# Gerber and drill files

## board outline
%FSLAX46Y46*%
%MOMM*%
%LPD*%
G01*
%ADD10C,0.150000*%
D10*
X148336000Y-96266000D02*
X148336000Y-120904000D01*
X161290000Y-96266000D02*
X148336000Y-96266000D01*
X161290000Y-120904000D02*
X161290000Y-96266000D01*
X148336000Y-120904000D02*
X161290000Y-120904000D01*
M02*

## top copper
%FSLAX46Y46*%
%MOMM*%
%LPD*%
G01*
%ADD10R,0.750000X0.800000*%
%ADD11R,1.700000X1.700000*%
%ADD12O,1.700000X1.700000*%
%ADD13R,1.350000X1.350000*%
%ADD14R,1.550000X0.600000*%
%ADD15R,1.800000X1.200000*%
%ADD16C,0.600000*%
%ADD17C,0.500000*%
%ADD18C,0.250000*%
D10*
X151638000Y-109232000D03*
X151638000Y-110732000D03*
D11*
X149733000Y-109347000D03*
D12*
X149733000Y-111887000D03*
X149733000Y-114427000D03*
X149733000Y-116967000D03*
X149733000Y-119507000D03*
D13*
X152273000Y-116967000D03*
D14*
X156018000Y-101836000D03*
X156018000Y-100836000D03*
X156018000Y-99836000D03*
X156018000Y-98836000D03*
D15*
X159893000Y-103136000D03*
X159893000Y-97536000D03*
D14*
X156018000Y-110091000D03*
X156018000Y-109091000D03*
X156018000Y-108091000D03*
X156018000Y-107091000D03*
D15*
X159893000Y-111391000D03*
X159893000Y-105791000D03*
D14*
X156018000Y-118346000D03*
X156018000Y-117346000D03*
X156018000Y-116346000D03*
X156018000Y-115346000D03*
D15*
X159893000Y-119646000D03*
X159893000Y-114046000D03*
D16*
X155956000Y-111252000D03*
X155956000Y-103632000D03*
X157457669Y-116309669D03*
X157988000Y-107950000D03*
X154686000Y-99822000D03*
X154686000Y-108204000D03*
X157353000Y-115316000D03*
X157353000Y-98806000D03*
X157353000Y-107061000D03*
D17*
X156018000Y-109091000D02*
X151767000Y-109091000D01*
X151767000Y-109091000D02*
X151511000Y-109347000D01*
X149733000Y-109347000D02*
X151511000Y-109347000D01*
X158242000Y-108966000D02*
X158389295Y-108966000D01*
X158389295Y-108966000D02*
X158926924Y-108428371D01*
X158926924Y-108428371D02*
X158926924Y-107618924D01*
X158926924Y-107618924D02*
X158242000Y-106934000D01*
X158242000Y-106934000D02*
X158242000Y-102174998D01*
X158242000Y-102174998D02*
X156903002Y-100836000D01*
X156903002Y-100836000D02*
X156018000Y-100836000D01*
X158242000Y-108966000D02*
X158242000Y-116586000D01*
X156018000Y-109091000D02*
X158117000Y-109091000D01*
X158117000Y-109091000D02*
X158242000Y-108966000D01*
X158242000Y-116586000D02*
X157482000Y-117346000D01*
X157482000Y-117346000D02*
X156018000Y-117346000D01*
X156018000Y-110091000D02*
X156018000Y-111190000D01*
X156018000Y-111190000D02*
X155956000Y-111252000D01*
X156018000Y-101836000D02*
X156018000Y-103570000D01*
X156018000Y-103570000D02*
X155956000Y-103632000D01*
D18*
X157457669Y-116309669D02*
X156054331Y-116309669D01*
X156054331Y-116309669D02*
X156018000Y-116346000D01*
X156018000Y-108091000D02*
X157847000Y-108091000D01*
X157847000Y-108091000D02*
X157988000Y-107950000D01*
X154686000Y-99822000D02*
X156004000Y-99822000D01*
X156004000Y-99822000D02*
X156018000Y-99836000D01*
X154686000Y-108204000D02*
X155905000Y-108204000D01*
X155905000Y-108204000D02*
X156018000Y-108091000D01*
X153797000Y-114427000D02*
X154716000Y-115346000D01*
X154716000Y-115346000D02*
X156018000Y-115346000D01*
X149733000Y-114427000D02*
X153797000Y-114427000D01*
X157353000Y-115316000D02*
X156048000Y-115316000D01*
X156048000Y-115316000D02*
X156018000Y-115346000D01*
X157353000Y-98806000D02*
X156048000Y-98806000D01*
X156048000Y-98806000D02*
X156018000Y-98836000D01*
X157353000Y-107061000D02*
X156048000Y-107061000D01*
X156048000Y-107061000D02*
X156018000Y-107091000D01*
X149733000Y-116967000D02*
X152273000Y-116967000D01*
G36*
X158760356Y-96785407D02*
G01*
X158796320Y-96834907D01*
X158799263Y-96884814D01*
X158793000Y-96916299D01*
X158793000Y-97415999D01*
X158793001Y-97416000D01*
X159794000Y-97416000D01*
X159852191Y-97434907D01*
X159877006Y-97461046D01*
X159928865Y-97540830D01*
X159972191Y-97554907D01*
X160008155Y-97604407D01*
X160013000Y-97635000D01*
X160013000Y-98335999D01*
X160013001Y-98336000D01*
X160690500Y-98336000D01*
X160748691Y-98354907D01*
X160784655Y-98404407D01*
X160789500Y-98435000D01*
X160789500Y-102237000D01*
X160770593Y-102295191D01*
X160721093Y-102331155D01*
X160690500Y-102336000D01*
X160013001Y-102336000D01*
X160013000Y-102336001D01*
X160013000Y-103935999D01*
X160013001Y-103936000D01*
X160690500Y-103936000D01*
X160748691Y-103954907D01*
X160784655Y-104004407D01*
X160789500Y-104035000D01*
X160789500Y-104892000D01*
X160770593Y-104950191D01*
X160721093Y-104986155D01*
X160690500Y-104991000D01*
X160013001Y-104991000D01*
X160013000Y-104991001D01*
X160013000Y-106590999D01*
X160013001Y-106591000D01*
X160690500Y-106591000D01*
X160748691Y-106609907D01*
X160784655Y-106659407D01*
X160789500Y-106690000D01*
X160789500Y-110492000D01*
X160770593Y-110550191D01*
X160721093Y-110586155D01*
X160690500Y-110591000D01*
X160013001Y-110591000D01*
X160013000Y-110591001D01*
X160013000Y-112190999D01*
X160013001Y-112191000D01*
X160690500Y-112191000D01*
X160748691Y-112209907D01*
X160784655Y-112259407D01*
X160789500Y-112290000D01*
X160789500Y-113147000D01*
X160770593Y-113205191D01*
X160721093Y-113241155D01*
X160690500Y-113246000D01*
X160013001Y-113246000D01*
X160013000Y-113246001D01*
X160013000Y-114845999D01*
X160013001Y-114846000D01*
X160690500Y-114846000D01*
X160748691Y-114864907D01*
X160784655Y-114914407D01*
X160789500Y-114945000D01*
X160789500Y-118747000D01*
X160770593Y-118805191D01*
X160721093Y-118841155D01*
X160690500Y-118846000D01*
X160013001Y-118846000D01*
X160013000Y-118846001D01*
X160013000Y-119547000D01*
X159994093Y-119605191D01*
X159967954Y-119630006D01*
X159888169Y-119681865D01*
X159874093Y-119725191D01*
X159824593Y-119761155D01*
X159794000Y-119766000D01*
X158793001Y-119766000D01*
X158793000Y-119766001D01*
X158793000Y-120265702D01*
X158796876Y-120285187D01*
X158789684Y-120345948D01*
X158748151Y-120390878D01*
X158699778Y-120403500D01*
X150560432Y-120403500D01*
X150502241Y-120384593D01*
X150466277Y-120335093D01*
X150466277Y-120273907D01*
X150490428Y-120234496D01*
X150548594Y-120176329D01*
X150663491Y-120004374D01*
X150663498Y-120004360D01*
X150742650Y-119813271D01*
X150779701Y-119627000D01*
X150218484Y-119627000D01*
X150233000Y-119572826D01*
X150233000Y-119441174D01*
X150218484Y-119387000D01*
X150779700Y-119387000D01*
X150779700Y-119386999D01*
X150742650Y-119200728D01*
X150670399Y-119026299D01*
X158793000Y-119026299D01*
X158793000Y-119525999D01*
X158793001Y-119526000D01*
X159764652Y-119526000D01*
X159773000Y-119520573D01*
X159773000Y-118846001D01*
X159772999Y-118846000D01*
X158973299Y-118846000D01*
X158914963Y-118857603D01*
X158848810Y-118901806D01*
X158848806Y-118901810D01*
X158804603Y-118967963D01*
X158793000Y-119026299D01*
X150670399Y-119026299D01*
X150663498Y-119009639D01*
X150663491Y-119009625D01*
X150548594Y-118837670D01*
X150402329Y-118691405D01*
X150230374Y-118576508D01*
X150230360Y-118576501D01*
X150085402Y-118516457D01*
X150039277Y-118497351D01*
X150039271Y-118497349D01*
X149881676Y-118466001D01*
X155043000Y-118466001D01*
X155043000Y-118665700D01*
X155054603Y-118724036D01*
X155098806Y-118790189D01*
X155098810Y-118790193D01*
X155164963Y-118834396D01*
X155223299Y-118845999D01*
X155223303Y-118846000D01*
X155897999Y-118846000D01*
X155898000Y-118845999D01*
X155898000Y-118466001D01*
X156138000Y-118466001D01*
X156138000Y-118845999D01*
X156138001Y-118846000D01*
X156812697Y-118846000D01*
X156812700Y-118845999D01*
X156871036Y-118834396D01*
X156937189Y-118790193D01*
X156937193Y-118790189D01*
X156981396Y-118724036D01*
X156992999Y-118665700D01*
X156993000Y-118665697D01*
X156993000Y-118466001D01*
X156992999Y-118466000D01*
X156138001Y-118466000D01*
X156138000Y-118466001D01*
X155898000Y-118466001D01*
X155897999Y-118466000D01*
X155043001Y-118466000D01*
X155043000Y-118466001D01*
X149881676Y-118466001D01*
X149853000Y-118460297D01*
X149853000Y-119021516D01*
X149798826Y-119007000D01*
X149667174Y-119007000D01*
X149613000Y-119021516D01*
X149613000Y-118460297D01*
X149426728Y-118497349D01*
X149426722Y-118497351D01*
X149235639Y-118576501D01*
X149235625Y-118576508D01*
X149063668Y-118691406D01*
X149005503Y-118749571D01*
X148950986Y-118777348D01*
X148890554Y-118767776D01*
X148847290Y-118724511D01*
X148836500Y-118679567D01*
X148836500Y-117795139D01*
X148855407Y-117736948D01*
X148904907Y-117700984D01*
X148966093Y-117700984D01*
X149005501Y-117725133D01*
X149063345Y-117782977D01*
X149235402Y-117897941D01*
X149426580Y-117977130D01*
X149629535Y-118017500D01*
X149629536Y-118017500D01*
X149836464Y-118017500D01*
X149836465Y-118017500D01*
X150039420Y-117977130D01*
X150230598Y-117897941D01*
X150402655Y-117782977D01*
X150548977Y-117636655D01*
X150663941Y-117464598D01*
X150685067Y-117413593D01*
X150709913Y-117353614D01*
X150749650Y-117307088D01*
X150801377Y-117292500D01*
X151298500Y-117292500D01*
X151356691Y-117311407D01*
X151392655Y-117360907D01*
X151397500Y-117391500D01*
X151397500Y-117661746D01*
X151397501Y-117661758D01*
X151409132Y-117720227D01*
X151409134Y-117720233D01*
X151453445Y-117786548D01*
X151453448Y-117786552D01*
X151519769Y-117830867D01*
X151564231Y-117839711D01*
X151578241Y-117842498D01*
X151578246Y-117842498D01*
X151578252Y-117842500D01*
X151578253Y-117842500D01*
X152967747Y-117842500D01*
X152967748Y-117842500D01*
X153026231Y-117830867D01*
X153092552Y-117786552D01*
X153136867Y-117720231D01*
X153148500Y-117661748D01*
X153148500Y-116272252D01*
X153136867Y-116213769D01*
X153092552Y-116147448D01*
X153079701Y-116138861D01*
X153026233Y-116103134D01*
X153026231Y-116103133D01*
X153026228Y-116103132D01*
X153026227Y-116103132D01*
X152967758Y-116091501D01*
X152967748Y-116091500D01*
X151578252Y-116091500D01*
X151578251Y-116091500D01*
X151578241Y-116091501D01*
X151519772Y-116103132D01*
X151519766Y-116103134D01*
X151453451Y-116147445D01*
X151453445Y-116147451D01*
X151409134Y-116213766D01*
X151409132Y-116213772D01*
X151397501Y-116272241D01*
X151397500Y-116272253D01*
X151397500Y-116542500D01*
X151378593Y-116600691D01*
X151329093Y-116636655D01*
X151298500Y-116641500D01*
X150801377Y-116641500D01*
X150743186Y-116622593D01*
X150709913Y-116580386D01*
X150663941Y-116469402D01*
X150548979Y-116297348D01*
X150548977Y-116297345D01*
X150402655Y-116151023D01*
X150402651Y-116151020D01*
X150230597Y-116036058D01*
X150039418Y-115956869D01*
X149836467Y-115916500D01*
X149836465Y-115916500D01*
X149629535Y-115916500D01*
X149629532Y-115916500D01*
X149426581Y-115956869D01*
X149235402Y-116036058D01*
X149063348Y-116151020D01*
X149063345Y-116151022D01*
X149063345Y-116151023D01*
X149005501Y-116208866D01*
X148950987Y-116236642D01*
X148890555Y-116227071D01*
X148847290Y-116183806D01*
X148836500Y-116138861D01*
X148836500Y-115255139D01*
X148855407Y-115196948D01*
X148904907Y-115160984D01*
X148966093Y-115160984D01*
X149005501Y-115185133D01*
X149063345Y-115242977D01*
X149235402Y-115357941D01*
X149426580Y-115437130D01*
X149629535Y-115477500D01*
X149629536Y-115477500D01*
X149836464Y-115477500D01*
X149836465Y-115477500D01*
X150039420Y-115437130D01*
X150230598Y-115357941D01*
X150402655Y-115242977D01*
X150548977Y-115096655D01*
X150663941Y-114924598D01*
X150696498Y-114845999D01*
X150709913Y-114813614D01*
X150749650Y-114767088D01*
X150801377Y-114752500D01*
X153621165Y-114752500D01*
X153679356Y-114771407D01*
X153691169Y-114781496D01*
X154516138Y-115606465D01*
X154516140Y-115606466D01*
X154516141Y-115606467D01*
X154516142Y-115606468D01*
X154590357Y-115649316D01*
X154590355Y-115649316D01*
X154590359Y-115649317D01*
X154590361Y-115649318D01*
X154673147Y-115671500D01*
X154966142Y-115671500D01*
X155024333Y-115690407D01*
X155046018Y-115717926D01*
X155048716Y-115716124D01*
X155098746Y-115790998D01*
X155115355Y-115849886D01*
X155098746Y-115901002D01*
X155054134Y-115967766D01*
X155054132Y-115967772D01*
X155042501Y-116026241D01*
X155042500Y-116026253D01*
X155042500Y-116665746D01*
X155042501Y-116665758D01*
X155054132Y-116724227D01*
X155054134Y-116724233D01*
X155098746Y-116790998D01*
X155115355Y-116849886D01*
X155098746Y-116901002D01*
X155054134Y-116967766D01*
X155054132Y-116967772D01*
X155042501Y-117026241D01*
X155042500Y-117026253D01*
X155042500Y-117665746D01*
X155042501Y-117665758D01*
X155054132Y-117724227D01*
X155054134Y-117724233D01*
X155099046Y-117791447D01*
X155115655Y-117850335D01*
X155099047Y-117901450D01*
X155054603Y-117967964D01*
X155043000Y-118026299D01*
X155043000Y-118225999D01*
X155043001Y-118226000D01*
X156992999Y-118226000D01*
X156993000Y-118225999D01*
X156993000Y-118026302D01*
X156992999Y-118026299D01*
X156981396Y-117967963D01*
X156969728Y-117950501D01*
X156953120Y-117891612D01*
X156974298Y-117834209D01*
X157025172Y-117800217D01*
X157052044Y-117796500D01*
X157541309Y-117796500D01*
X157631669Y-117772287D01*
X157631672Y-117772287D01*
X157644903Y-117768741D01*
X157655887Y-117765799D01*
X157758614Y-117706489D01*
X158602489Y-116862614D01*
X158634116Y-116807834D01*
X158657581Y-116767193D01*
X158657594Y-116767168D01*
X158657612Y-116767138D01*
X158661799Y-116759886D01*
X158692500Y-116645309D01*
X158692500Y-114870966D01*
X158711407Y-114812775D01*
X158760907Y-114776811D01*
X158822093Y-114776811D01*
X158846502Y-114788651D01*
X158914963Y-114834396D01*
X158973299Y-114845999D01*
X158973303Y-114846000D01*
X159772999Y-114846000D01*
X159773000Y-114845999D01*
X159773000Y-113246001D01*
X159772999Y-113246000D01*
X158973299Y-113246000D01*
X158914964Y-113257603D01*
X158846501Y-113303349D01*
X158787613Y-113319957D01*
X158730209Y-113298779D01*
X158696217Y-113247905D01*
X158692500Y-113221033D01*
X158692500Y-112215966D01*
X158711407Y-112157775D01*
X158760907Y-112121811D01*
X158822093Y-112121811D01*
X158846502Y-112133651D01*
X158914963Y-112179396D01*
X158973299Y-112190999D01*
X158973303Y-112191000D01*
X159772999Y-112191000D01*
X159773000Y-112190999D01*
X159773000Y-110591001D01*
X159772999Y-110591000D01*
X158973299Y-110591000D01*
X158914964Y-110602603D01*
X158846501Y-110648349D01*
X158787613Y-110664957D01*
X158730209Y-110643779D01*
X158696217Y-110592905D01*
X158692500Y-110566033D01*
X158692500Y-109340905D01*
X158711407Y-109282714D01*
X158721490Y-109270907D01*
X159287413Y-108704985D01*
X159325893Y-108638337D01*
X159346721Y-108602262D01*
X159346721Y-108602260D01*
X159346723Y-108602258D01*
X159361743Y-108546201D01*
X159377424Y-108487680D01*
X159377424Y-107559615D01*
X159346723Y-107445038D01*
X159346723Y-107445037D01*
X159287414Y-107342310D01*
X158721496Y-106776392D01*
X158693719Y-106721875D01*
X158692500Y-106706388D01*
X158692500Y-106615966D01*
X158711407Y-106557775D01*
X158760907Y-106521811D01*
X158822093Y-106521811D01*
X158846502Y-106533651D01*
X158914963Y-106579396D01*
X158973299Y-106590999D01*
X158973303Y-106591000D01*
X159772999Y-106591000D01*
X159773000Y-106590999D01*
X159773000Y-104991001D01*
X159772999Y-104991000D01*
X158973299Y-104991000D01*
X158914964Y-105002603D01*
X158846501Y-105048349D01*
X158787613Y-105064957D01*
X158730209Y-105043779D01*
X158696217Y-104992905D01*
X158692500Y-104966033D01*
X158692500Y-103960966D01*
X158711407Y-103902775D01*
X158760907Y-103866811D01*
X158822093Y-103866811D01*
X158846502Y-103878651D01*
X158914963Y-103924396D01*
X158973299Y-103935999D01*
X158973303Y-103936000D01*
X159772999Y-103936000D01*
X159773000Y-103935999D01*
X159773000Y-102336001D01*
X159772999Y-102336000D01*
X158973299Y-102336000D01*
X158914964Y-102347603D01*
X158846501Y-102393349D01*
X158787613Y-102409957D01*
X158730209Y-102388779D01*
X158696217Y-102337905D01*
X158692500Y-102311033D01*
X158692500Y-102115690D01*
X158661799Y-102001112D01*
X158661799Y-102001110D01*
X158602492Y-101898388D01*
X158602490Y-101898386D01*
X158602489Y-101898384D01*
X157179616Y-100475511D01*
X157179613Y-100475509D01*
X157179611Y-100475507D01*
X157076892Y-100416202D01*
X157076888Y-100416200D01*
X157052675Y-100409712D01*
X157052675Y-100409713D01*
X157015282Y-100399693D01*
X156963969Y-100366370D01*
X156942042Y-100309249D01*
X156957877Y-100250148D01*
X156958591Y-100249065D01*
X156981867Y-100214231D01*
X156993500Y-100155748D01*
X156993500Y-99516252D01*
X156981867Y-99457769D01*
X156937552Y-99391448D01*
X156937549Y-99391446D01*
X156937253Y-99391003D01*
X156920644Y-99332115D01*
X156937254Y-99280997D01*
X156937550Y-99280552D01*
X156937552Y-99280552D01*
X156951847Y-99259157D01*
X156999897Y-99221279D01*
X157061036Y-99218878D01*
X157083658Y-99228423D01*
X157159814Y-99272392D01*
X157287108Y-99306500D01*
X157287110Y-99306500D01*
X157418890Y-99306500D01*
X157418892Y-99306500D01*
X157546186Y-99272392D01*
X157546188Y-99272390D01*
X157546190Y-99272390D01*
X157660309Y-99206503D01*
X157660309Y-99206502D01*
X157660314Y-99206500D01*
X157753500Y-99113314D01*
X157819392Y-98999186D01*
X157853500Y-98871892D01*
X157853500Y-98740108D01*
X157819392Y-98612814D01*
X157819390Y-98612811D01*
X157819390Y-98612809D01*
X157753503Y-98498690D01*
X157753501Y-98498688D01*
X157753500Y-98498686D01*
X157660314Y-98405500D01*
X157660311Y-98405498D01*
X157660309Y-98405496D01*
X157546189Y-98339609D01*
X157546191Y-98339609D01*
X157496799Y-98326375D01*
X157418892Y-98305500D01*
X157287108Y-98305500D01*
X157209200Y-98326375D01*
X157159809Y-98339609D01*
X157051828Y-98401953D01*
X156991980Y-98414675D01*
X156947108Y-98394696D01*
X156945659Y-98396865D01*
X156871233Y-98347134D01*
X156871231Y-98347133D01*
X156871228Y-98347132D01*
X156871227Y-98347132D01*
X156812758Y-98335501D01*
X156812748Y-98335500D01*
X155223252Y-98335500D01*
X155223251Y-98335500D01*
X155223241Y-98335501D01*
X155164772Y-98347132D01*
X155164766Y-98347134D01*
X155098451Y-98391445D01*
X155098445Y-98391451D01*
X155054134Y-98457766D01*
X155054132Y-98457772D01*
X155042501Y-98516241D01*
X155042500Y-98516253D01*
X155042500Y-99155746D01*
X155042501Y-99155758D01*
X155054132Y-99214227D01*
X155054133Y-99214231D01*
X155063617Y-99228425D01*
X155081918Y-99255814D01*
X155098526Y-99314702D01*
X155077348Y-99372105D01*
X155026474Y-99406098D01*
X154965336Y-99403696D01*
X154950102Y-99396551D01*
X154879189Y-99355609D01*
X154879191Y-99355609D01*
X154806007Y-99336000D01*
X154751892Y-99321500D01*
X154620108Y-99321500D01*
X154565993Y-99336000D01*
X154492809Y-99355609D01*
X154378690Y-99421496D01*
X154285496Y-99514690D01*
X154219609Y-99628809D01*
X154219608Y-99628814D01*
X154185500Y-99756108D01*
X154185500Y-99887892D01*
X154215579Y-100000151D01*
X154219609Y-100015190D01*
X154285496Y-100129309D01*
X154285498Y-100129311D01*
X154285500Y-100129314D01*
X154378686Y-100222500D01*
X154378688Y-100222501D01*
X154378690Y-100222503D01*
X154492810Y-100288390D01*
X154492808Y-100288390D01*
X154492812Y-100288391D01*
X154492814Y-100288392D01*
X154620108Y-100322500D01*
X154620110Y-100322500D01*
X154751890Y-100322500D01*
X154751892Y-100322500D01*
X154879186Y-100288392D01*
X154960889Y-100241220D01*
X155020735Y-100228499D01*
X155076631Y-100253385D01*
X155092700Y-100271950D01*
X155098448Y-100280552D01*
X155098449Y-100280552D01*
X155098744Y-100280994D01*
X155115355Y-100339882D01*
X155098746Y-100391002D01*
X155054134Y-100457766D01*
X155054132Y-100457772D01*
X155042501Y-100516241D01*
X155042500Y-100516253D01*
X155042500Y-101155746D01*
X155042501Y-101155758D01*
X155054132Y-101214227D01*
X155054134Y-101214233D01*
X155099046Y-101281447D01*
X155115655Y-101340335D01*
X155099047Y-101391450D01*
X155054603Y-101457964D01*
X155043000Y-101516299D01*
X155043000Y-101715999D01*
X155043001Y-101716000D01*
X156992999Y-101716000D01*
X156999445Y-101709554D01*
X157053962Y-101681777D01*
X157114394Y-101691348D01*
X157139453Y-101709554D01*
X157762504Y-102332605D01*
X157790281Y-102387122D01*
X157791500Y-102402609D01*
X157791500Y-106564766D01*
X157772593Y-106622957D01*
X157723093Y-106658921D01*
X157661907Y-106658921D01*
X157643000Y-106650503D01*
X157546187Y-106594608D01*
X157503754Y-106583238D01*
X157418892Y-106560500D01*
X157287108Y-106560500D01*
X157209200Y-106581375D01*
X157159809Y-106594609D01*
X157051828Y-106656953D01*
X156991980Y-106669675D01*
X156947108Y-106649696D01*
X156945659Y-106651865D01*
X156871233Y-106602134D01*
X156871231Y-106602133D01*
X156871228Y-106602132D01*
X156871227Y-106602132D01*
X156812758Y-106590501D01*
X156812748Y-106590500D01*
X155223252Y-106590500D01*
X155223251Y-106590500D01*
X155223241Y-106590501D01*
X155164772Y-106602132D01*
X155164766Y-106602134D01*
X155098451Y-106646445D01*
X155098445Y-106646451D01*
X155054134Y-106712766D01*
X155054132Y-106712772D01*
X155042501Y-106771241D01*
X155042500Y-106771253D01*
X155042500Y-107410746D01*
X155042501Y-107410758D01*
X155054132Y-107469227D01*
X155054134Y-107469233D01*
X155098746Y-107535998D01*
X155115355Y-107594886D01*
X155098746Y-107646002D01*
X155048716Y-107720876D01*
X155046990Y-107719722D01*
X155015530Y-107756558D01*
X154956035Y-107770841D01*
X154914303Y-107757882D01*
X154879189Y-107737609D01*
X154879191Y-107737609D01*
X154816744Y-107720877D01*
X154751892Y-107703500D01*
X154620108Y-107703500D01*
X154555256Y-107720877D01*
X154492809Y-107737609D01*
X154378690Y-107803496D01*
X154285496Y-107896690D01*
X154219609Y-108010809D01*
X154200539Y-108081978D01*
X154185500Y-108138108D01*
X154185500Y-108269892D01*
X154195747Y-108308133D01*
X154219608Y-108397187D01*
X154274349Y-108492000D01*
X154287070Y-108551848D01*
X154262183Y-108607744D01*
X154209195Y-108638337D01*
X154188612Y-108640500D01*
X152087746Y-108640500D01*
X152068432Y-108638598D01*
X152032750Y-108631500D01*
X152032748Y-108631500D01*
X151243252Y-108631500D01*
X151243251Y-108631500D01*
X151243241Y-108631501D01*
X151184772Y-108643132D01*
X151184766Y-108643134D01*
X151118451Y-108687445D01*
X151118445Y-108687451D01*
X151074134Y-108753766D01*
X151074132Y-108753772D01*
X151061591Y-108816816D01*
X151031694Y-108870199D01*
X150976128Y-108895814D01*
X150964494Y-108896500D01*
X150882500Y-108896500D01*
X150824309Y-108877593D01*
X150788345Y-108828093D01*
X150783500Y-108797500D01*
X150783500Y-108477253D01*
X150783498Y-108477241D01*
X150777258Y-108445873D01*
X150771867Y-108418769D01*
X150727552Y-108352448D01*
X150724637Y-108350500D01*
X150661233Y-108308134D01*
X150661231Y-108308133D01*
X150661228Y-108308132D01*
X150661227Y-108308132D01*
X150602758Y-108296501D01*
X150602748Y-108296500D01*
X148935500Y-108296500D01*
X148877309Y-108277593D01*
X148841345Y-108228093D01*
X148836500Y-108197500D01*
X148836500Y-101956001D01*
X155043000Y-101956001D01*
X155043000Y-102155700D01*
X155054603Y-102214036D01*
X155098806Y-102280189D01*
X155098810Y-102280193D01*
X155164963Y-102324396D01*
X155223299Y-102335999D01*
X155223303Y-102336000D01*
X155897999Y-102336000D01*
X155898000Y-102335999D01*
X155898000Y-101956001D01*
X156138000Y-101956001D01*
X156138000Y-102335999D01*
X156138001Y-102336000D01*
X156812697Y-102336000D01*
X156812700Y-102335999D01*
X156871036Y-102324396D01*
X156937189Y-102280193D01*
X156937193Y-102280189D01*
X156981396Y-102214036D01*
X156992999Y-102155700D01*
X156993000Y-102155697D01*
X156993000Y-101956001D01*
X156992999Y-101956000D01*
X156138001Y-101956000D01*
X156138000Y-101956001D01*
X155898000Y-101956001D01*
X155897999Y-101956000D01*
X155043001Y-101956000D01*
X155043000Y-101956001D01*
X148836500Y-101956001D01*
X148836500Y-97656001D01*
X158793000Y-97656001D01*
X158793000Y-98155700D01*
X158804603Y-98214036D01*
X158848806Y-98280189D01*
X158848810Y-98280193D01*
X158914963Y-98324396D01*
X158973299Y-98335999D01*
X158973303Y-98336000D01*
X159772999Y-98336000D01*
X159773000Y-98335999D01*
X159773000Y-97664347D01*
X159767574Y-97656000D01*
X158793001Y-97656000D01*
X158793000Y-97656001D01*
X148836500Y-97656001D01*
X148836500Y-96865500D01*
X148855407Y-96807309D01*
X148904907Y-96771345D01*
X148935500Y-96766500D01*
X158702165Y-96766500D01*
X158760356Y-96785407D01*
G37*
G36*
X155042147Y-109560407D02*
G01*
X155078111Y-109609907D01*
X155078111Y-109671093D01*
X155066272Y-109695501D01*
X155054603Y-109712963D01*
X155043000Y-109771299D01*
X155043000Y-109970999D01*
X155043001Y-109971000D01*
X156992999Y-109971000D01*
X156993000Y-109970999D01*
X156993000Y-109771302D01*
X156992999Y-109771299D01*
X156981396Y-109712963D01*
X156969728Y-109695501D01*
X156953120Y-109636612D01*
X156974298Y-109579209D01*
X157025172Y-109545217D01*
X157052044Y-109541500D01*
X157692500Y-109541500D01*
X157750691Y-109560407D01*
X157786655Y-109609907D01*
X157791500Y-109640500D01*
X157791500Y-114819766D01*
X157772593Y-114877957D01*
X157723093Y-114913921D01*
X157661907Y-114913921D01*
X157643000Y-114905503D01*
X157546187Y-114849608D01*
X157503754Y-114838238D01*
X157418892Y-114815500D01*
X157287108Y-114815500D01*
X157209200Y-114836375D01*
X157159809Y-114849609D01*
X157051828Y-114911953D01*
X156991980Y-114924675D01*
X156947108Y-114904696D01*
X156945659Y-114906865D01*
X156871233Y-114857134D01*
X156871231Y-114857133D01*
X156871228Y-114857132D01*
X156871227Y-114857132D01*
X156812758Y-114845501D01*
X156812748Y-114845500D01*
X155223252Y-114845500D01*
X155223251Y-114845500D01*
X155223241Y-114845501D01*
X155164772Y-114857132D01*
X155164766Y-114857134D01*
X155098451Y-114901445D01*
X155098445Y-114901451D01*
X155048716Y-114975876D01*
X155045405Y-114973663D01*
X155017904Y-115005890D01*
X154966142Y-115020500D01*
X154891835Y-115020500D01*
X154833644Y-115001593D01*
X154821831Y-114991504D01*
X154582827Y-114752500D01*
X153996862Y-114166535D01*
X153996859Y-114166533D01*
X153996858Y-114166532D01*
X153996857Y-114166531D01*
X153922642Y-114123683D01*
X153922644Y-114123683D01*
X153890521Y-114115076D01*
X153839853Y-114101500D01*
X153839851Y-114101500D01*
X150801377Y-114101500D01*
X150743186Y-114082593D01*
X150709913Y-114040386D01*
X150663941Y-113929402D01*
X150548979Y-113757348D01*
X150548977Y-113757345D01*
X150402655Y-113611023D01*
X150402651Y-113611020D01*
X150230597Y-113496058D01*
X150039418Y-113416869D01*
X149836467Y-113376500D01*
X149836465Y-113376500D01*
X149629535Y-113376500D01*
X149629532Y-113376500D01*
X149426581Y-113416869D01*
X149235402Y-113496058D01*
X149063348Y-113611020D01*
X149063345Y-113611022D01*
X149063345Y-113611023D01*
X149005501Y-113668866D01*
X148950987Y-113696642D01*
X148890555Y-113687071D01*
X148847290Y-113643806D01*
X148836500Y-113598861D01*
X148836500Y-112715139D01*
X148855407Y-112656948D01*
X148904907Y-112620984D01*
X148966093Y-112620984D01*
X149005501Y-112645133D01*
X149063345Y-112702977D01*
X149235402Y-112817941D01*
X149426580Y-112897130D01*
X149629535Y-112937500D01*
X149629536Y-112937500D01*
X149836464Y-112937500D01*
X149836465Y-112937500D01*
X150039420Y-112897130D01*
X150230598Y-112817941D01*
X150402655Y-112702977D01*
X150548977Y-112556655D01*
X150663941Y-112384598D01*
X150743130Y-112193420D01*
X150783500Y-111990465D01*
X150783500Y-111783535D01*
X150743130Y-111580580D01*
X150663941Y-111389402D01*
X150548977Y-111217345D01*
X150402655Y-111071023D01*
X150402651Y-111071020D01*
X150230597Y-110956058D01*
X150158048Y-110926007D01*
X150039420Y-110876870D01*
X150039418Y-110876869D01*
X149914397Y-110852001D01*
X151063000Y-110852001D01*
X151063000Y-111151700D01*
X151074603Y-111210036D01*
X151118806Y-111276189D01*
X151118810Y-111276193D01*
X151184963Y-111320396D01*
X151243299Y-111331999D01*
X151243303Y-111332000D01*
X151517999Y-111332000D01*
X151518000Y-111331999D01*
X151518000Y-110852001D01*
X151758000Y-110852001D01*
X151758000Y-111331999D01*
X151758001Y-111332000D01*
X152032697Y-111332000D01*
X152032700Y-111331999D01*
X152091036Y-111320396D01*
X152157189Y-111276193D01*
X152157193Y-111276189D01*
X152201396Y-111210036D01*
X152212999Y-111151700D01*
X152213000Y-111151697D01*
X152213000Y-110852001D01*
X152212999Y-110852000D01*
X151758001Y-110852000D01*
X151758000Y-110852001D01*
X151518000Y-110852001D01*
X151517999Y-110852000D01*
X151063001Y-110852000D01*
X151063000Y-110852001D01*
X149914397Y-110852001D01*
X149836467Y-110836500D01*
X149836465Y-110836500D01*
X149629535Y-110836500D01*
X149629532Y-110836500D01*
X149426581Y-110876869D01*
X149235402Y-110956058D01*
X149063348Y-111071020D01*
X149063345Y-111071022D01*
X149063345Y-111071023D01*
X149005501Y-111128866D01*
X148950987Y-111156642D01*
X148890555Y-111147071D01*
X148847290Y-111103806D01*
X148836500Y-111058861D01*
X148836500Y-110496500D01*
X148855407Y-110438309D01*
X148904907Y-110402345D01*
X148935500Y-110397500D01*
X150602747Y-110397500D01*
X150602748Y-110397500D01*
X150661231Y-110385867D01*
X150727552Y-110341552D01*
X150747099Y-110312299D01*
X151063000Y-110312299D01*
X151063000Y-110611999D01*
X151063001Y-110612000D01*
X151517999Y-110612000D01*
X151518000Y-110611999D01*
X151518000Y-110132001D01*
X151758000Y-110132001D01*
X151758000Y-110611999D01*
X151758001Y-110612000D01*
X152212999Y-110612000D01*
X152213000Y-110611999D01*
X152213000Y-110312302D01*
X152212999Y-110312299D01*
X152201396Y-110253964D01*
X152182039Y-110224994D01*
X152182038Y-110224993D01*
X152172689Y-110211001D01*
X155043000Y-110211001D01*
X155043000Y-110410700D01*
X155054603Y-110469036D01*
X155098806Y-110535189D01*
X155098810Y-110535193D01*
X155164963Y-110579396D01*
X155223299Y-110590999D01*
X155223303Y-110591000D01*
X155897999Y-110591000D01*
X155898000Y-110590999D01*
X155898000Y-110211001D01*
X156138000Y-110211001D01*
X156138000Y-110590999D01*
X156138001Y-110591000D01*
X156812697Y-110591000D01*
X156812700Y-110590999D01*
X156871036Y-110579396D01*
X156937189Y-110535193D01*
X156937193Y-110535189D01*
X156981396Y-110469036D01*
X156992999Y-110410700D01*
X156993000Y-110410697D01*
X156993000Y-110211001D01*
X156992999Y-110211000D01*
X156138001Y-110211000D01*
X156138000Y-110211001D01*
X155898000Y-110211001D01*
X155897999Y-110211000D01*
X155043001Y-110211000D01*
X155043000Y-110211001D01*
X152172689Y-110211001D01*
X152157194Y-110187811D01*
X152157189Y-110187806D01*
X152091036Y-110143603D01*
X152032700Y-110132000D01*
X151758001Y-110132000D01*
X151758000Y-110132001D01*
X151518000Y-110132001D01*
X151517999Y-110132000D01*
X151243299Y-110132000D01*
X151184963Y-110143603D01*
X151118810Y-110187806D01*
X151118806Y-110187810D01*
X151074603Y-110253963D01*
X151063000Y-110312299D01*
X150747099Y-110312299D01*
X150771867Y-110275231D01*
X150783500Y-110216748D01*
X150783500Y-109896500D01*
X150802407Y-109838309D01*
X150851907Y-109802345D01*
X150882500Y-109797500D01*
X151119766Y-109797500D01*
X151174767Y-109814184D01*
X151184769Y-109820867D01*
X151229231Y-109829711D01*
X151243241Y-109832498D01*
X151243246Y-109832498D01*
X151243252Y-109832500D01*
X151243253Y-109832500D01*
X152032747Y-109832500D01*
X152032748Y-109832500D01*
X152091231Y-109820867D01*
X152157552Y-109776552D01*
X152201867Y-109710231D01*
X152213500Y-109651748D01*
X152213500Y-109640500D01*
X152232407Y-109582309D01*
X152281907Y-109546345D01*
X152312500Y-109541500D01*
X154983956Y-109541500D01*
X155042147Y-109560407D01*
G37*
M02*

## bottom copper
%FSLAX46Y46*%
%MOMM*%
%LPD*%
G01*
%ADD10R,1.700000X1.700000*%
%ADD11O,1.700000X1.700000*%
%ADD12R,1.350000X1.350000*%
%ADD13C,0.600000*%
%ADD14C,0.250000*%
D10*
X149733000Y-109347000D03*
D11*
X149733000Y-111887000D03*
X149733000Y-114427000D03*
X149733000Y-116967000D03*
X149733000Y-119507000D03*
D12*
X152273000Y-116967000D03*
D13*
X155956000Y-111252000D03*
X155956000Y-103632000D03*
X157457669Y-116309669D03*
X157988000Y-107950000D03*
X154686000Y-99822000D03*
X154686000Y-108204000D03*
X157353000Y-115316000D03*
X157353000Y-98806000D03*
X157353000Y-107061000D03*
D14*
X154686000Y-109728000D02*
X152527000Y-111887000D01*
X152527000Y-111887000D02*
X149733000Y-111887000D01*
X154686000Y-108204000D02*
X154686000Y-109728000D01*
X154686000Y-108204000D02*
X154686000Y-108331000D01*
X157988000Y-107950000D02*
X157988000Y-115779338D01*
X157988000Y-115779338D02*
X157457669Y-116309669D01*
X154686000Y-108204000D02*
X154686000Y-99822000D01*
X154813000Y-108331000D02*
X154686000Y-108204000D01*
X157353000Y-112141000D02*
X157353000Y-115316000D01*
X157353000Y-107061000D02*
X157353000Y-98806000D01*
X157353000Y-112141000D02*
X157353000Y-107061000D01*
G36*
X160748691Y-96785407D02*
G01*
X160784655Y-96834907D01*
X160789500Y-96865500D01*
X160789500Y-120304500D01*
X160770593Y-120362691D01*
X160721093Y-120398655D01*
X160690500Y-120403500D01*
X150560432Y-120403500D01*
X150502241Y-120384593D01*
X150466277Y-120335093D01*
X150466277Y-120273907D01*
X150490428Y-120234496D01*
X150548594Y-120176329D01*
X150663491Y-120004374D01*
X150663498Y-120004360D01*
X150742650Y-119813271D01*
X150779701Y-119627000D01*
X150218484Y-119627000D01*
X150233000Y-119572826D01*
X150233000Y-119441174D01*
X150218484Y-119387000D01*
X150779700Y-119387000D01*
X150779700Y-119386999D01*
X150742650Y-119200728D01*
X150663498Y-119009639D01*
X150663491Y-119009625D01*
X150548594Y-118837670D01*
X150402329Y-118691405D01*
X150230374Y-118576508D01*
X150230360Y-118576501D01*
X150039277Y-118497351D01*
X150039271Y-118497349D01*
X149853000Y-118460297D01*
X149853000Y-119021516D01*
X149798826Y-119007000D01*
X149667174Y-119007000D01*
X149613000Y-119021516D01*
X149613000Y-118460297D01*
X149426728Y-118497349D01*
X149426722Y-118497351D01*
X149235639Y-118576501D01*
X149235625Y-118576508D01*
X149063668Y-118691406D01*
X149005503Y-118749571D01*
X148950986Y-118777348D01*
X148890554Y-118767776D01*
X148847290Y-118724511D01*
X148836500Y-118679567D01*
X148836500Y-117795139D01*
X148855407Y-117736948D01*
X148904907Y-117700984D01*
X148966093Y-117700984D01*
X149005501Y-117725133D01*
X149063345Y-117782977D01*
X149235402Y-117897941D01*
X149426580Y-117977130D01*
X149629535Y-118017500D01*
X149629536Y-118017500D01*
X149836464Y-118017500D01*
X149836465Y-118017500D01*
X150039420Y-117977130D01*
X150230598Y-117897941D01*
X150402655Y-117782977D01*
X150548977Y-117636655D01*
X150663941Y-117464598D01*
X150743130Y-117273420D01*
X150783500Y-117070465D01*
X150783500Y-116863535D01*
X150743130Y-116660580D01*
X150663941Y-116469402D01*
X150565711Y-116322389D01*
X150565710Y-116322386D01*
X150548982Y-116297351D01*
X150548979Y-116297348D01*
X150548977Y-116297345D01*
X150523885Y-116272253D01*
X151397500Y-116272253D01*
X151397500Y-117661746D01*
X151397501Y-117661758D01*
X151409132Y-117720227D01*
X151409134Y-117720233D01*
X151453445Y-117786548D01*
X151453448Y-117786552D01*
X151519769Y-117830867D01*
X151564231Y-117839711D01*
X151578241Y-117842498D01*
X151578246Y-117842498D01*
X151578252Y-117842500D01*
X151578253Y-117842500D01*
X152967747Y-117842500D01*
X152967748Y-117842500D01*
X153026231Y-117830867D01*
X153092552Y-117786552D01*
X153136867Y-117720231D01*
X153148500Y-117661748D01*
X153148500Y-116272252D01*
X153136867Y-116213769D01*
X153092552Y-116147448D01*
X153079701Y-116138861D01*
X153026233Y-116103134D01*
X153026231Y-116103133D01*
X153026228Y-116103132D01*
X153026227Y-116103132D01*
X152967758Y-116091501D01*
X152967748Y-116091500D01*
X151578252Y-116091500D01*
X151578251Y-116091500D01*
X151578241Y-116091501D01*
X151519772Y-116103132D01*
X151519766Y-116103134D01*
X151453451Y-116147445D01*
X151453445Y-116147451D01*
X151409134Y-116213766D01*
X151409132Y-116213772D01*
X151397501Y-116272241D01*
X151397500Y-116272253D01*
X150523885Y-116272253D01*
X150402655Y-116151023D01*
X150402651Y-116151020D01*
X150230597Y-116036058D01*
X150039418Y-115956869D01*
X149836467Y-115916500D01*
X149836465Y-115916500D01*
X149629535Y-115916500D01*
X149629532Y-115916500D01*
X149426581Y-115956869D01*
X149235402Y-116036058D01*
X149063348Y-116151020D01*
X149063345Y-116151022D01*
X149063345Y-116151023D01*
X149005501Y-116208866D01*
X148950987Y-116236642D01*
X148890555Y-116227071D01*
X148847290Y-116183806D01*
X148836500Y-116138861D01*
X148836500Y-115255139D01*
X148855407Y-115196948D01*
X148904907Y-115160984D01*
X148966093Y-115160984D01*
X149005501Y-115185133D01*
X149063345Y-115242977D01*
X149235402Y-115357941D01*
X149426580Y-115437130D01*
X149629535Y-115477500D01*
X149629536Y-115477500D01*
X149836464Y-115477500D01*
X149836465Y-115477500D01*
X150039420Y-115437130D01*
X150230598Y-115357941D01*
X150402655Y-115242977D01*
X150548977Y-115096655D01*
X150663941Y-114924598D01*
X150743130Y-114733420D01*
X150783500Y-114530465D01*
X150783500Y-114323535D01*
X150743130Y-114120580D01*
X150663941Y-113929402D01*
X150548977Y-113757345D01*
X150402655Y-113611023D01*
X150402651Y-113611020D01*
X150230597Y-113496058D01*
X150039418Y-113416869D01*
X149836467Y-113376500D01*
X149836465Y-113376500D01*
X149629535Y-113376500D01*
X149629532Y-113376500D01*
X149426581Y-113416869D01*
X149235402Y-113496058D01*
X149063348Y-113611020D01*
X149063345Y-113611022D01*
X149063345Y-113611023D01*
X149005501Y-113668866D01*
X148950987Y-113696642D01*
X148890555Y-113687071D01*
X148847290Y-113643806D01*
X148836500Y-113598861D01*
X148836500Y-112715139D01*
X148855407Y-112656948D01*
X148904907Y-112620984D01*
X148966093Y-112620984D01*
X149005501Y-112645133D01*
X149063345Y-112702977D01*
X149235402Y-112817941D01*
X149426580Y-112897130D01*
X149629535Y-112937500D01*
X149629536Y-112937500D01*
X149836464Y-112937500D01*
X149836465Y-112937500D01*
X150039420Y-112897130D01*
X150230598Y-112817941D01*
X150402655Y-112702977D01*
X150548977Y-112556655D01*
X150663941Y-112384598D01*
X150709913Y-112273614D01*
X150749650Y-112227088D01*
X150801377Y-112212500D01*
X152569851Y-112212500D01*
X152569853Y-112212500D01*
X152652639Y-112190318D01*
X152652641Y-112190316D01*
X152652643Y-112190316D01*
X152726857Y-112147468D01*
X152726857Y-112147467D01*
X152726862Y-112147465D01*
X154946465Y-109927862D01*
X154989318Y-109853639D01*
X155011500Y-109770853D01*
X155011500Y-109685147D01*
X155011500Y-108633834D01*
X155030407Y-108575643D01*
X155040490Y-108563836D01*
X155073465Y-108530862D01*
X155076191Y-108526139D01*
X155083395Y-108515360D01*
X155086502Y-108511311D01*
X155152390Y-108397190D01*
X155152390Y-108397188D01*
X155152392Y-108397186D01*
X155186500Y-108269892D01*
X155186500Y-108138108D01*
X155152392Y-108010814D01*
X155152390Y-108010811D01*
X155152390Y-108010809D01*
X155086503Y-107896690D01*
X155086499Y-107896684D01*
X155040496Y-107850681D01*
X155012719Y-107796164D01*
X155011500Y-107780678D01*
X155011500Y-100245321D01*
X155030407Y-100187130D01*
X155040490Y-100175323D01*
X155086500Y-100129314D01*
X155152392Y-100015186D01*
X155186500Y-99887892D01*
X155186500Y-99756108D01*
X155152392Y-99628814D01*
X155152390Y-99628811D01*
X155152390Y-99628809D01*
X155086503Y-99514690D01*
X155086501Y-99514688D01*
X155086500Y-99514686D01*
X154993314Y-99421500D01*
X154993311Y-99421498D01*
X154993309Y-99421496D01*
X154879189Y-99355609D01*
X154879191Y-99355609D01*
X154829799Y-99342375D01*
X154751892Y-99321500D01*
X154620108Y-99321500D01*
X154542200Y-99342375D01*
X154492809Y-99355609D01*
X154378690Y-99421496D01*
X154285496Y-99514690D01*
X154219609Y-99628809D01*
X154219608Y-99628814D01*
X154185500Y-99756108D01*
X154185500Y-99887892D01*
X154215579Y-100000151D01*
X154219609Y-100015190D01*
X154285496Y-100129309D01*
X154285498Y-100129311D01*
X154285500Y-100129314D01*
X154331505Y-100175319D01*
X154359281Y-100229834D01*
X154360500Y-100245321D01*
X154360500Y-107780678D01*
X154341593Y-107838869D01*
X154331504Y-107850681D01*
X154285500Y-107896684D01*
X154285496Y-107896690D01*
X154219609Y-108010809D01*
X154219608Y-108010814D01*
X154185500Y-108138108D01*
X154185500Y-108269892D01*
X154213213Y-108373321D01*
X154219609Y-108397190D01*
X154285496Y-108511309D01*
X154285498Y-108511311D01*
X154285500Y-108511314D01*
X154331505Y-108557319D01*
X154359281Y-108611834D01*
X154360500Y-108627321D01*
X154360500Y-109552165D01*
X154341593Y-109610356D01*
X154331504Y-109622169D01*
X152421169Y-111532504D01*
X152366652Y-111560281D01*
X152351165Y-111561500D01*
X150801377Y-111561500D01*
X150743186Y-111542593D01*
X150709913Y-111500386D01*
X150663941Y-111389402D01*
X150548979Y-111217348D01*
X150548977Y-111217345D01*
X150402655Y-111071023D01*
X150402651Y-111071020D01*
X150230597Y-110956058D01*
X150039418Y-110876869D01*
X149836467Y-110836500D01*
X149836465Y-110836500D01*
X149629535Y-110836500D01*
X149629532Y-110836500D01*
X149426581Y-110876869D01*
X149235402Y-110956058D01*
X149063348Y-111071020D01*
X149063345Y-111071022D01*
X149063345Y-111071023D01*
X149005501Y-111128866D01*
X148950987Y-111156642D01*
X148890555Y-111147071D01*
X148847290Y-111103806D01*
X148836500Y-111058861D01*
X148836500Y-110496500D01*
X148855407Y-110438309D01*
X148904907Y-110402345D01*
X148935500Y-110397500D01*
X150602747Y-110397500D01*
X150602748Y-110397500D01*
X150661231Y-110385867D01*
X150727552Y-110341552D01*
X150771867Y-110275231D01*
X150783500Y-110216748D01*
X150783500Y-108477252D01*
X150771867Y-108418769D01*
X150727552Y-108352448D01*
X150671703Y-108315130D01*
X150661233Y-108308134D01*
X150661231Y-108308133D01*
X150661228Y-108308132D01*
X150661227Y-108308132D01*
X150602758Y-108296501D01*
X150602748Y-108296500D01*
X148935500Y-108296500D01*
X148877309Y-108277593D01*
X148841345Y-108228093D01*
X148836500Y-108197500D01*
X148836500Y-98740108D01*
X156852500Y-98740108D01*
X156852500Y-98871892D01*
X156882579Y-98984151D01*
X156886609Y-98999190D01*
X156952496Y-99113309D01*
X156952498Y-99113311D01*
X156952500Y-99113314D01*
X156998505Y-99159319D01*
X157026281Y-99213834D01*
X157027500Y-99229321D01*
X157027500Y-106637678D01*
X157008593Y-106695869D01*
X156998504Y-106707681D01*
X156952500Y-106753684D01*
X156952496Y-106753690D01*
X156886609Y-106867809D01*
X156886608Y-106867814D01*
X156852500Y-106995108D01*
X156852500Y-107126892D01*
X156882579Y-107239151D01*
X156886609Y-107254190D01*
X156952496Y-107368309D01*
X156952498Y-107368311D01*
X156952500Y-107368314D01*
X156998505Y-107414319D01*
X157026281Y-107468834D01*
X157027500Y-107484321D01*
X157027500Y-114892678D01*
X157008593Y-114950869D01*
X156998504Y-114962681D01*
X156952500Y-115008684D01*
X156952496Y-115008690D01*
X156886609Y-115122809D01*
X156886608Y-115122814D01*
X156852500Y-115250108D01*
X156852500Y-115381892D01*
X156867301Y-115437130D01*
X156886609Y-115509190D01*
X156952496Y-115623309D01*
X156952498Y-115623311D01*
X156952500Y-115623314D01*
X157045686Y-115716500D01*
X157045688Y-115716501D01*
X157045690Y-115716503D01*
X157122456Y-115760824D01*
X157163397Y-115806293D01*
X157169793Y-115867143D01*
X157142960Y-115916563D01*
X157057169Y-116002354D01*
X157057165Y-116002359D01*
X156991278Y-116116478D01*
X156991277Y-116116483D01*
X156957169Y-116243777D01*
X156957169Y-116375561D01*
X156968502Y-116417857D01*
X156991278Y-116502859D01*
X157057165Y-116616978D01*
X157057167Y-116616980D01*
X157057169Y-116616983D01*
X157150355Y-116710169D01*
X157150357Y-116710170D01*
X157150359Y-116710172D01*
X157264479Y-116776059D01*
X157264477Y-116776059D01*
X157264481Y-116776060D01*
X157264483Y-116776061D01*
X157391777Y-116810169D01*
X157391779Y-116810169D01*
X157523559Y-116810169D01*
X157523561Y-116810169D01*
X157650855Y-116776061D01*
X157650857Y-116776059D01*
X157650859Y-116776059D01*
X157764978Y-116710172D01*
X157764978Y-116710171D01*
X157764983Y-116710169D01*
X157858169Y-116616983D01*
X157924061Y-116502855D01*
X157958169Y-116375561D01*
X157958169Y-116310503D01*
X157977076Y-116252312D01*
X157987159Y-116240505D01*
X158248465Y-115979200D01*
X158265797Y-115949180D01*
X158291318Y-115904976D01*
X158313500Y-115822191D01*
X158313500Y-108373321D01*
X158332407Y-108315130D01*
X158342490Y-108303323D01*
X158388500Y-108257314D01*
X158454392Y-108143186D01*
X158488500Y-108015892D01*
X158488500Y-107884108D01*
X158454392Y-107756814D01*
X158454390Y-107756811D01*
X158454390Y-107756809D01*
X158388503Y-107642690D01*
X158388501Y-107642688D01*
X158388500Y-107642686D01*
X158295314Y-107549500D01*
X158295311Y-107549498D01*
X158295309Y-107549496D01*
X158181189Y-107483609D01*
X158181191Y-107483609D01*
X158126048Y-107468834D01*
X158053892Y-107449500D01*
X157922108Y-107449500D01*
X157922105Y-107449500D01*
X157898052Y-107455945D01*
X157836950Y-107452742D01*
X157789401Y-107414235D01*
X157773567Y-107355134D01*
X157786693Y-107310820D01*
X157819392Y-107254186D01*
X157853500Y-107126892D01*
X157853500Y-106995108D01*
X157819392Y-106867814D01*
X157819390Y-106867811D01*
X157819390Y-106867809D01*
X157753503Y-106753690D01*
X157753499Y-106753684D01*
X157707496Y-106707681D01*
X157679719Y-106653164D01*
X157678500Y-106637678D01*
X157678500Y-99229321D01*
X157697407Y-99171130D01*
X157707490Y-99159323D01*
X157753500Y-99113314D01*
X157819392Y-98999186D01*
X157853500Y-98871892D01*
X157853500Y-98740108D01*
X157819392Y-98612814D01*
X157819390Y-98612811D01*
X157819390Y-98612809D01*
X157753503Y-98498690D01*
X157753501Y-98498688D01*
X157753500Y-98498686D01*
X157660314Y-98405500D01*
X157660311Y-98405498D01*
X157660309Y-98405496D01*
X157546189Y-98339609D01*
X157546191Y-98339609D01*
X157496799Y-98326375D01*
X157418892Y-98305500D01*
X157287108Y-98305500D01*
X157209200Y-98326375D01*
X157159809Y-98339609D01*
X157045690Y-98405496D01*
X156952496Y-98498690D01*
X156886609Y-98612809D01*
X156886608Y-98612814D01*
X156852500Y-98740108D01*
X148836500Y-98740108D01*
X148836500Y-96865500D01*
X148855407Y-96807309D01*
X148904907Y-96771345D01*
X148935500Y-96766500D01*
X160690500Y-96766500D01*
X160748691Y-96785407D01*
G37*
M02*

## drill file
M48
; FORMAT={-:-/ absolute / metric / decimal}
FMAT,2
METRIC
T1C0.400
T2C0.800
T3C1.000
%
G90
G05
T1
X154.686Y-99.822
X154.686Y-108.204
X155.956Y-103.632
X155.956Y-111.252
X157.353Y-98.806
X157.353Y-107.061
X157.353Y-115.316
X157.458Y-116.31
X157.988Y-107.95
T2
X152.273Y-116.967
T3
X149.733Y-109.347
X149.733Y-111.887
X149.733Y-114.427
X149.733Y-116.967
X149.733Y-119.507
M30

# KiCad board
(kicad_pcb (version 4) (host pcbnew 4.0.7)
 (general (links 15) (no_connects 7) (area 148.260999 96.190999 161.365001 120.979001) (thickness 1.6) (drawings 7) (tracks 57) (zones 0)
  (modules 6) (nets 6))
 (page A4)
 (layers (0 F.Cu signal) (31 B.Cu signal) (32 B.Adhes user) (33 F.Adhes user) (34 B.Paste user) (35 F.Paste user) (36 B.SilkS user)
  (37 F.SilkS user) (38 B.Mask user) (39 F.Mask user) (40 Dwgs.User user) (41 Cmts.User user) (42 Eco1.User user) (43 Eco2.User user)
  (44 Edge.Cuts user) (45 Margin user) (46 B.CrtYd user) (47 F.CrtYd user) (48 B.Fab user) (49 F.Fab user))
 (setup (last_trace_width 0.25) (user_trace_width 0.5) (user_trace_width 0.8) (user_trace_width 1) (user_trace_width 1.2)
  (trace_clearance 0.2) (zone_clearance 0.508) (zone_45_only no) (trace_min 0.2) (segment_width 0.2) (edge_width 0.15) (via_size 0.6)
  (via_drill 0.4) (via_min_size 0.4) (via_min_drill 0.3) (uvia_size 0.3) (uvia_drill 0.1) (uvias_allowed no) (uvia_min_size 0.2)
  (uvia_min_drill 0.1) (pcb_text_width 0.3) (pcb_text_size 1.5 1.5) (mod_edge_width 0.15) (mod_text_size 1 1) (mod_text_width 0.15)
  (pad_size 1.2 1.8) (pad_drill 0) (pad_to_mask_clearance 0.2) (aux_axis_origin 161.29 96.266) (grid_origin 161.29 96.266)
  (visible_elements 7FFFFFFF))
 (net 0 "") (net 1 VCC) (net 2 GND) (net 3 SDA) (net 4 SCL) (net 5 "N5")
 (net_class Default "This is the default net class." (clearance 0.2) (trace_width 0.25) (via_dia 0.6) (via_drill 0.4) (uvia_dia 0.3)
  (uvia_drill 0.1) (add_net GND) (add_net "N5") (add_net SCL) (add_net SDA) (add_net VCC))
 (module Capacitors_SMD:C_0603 (layer F.Cu) (at 151.638 109.982 90)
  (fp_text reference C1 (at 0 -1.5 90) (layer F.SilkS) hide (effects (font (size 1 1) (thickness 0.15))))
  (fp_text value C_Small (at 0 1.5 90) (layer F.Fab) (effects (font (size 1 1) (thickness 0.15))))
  (pad 2 smd rect (at 0.75 0 90) (size 0.8 0.75) (layers F.Cu F.Paste F.Mask) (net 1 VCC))
  (pad 1 smd rect (at -0.75 0 90) (size 0.8 0.75) (layers F.Cu F.Paste F.Mask) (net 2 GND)))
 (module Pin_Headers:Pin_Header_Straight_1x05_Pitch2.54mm (layer F.Cu) (at 149.733 109.347)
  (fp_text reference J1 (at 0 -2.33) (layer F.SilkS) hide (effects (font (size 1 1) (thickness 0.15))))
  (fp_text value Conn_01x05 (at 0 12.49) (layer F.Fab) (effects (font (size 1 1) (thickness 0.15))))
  (pad 1 thru_hole rect (at 0 0) (size 1.7 1.7) (drill 1) (layers *.Cu *.Mask) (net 1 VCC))
  (pad 2 thru_hole oval (at 0 2.54) (size 1.7 1.7) (drill 1) (layers *.Cu *.Mask) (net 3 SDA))
  (pad 3 thru_hole oval (at 0 5.08) (size 1.7 1.7) (drill 1) (layers *.Cu *.Mask) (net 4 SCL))
  (pad 4 thru_hole oval (at 0 7.62) (size 1.7 1.7) (drill 1) (layers *.Cu *.Mask) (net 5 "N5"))
  (pad 5 thru_hole oval (at 0 10.16) (size 1.7 1.7) (drill 1) (layers *.Cu *.Mask) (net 2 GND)))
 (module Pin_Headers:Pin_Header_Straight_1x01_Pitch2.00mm (layer F.Cu) (at 152.273 116.967)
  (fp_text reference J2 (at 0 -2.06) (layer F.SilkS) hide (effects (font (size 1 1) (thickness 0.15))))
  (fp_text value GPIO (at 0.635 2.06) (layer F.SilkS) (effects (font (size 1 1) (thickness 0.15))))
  (pad 1 thru_hole rect (at 0 0) (size 1.35 1.35) (drill 0.8) (layers *.Cu *.Mask) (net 5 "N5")))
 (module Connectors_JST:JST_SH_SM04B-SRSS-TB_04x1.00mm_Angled (layer F.Cu) (at 157.9555 100.336 90)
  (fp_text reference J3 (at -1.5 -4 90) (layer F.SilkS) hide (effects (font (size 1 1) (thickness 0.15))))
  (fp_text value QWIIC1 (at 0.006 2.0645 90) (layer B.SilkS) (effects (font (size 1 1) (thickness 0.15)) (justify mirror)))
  (pad 1 smd rect (at -1.5 -1.9375 90) (size 0.6 1.55) (layers F.Cu F.Paste F.Mask) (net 2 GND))
  (pad 2 smd rect (at -0.5 -1.9375 90) (size 0.6 1.55) (layers F.Cu F.Paste F.Mask) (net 1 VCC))
  (pad 3 smd rect (at 0.5 -1.9375 90) (size 0.6 1.55) (layers F.Cu F.Paste F.Mask) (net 3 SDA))
  (pad 4 smd rect (at 1.5 -1.9375 90) (size 0.6 1.55) (layers F.Cu F.Paste F.Mask) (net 4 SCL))
  (pad "" smd rect (at -2.8 1.9375 90) (size 1.2 1.8) (layers F.Cu F.Paste F.Mask) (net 2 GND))
  (pad "" smd rect (at 2.8 1.9375 90) (size 1.2 1.8) (layers F.Cu F.Paste F.Mask) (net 2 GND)))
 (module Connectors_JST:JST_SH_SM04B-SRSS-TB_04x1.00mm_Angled (layer F.Cu) (at 157.9555 108.591 90)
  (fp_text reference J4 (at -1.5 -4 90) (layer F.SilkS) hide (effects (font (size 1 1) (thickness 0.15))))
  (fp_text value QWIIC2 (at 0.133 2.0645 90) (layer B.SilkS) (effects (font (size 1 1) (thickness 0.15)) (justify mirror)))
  (pad 1 smd rect (at -1.5 -1.9375 90) (size 0.6 1.55) (layers F.Cu F.Paste F.Mask) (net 2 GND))
  (pad 2 smd rect (at -0.5 -1.9375 90) (size 0.6 1.55) (layers F.Cu F.Paste F.Mask) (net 1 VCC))
  (pad 3 smd rect (at 0.5 -1.9375 90) (size 0.6 1.55) (layers F.Cu F.Paste F.Mask) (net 3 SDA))
  (pad 4 smd rect (at 1.5 -1.9375 90) (size 0.6 1.55) (layers F.Cu F.Paste F.Mask) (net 4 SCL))
  (pad "" smd rect (at -2.8 1.9375 90) (size 1.2 1.8) (layers F.Cu F.Paste F.Mask) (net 2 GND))
  (pad "" smd rect (at 2.8 1.9375 90) (size 1.2 1.8) (layers F.Cu F.Paste F.Mask) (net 2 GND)))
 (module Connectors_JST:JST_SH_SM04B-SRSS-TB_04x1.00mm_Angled (layer F.Cu) (at 157.9555 116.846 90)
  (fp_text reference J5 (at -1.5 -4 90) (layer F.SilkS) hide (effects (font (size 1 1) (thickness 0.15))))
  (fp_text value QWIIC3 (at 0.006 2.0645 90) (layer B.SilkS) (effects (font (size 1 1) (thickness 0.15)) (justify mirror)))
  (pad 1 smd rect (at -1.5 -1.9375 90) (size 0.6 1.55) (layers F.Cu F.Paste F.Mask) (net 2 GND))
  (pad 2 smd rect (at -0.5 -1.9375 90) (size 0.6 1.55) (layers F.Cu F.Paste F.Mask) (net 1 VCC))
  (pad 3 smd rect (at 0.5 -1.9375 90) (size 0.6 1.55) (layers F.Cu F.Paste F.Mask) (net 3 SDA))
  (pad 4 smd rect (at 1.5 -1.9375 90) (size 0.6 1.55) (layers F.Cu F.Paste F.Mask) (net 4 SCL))
  (pad "" smd rect (at -2.8 1.9375 90) (size 1.2 1.8) (layers F.Cu F.Paste F.Mask) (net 2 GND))
  (pad "" smd rect (at 2.8 1.9375 90) (size 1.2 1.8) (layers F.Cu F.Paste F.Mask) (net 2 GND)))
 (gr_line (start 148.336 96.266) (end 148.336 120.904) (layer Edge.Cuts) (width 0.15))
 (gr_line (start 161.29 96.266) (end 148.336 96.266) (layer Edge.Cuts) (width 0.15))
 (gr_line (start 161.29 120.904) (end 161.29 96.266) (layer Edge.Cuts) (width 0.15))
 (gr_line (start 148.336 120.904) (end 161.29 120.904) (layer Edge.Cuts) (width 0.15))
 (segment (start 156.018 109.091) (end 151.767 109.091) (width 0.5) (layer F.Cu) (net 1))
 (segment (start 151.767 109.091) (end 151.511 109.347) (width 0.5) (layer F.Cu) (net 1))
 (segment (start 149.733 109.347) (end 151.511 109.347) (width 0.5) (layer F.Cu) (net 1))
 (segment (start 158.242 108.966) (end 158.389295 108.966) (width 0.5) (layer F.Cu) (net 1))
 (segment (start 158.389295 108.966) (end 158.926924 108.428371) (width 0.5) (layer F.Cu) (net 1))
 (segment (start 158.926924 108.428371) (end 158.926924 107.618924) (width 0.5) (layer F.Cu) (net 1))
 (segment (start 158.926924 107.618924) (end 158.242 106.934) (width 0.5) (layer F.Cu) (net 1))
 (segment (start 158.242 106.934) (end 158.242 102.174998) (width 0.5) (layer F.Cu) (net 1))
 (segment (start 158.242 102.174998) (end 156.903002 100.836) (width 0.5) (layer F.Cu) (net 1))
 (segment (start 156.903002 100.836) (end 156.018 100.836) (width 0.5) (layer F.Cu) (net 1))
 (segment (start 158.242 108.966) (end 158.242 116.586) (width 0.5) (layer F.Cu) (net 1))
 (segment (start 156.018 109.091) (end 158.117 109.091) (width 0.5) (layer F.Cu) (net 1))
 (segment (start 158.117 109.091) (end 158.242 108.966) (width 0.5) (layer F.Cu) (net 1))
 (segment (start 158.242 116.586) (end 157.482 117.346) (width 0.5) (layer F.Cu) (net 1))
 (segment (start 157.482 117.346) (end 156.018 117.346) (width 0.5) (layer F.Cu) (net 1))
 (segment (start 156.018 110.091) (end 156.018 111.19) (width 0.5) (layer F.Cu) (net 2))
 (segment (start 156.018 111.19) (end 155.956 111.252) (width 0.5) (layer F.Cu) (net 2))
 (via (at 155.956 111.252) (size 0.6) (drill 0.4) (layers F.Cu B.Cu) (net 2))
 (segment (start 156.018 101.836) (end 156.018 103.57) (width 0.5) (layer F.Cu) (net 2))
 (segment (start 156.018 103.57) (end 155.956 103.632) (width 0.5) (layer F.Cu) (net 2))
 (via (at 155.956 103.632) (size 0.6) (drill 0.4) (layers F.Cu B.Cu) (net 2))
 (segment (start 154.686 109.728) (end 152.527 111.887) (width 0.25) (layer B.Cu) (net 3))
 (segment (start 152.527 111.887) (end 149.733 111.887) (width 0.25) (layer B.Cu) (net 3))
 (segment (start 154.686 108.204) (end 154.686 109.728) (width 0.25) (layer B.Cu) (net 3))
 (segment (start 154.686 108.204) (end 154.686 108.331) (width 0.25) (layer B.Cu) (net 3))
 (segment (start 157.457669 116.309669) (end 156.054331 116.309669) (width 0.25) (layer F.Cu) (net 3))
 (segment (start 156.054331 116.309669) (end 156.018 116.346) (width 0.25) (layer F.Cu) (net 3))
 (segment (start 157.988 107.95) (end 157.988 115.779338) (width 0.25) (layer B.Cu) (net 3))
 (segment (start 157.988 115.779338) (end 157.457669 116.309669) (width 0.25) (layer B.Cu) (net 3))
 (via (at 157.457669 116.309669) (size 0.6) (drill 0.4) (layers F.Cu B.Cu) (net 3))
 (segment (start 156.018 108.091) (end 157.847 108.091) (width 0.25) (layer F.Cu) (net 3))
 (segment (start 157.847 108.091) (end 157.988 107.95) (width 0.25) (layer F.Cu) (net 3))
 (via (at 157.988 107.95) (size 0.6) (drill 0.4) (layers F.Cu B.Cu) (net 3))
 (segment (start 154.686 99.822) (end 156.004 99.822) (width 0.25) (layer F.Cu) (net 3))
 (segment (start 156.004 99.822) (end 156.018 99.836) (width 0.25) (layer F.Cu) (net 3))
 (segment (start 154.686 108.204) (end 154.686 99.822) (width 0.25) (layer B.Cu) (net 3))
 (via (at 154.686 99.822) (size 0.6) (drill 0.4) (layers F.Cu B.Cu) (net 3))
 (segment (start 154.686 108.204) (end 155.905 108.204) (width 0.25) (layer F.Cu) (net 3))
 (segment (start 155.905 108.204) (end 156.018 108.091) (width 0.25) (layer F.Cu) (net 3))
 (segment (start 154.813 108.331) (end 154.686 108.204) (width 0.25) (layer B.Cu) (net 3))
 (via (at 154.686 108.204) (size 0.6) (drill 0.4) (layers F.Cu B.Cu) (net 3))
 (segment (start 153.797 114.427) (end 154.716 115.346) (width 0.25) (layer F.Cu) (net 4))
 (segment (start 154.716 115.346) (end 156.018 115.346) (width 0.25) (layer F.Cu) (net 4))
 (segment (start 149.733 114.427) (end 153.797 114.427) (width 0.25) (layer F.Cu) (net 4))
 (segment (start 157.353 115.316) (end 156.048 115.316) (width 0.25) (layer F.Cu) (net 4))
 (segment (start 156.048 115.316) (end 156.018 115.346) (width 0.25) (layer F.Cu) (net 4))
 (segment (start 157.353 112.141) (end 157.353 115.316) (width 0.25) (layer B.Cu) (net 4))
 (via (at 157.353 115.316) (size 0.6) (drill 0.4) (layers F.Cu B.Cu) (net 4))
 (segment (start 157.353 98.806) (end 156.048 98.806) (width 0.25) (layer F.Cu) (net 4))
 (segment (start 156.048 98.806) (end 156.018 98.836) (width 0.25) (layer F.Cu) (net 4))
 (segment (start 157.353 107.061) (end 157.353 98.806) (width 0.25) (layer B.Cu) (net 4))
 (via (at 157.353 98.806) (size 0.6) (drill 0.4) (layers F.Cu B.Cu) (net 4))
 (segment (start 157.353 107.061) (end 156.048 107.061) (width 0.25) (layer F.Cu) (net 4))
 (segment (start 156.048 107.061) (end 156.018 107.091) (width 0.25) (layer F.Cu) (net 4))
 (segment (start 157.353 112.141) (end 157.353 107.061) (width 0.25) (layer B.Cu) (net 4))
 (via (at 157.353 107.061) (size 0.6) (drill 0.4) (layers F.Cu B.Cu) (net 4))
 (segment (start 149.733 116.967) (end 152.273 116.967) (width 0.25) (layer F.Cu) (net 5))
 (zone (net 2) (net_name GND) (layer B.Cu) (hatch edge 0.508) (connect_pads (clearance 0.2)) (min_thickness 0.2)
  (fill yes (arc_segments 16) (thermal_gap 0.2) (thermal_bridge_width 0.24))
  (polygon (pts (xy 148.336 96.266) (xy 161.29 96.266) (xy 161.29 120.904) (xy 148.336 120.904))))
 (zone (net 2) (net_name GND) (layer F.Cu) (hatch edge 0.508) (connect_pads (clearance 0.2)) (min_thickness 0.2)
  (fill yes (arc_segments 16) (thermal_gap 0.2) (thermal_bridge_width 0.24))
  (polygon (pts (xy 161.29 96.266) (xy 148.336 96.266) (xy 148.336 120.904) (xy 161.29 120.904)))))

